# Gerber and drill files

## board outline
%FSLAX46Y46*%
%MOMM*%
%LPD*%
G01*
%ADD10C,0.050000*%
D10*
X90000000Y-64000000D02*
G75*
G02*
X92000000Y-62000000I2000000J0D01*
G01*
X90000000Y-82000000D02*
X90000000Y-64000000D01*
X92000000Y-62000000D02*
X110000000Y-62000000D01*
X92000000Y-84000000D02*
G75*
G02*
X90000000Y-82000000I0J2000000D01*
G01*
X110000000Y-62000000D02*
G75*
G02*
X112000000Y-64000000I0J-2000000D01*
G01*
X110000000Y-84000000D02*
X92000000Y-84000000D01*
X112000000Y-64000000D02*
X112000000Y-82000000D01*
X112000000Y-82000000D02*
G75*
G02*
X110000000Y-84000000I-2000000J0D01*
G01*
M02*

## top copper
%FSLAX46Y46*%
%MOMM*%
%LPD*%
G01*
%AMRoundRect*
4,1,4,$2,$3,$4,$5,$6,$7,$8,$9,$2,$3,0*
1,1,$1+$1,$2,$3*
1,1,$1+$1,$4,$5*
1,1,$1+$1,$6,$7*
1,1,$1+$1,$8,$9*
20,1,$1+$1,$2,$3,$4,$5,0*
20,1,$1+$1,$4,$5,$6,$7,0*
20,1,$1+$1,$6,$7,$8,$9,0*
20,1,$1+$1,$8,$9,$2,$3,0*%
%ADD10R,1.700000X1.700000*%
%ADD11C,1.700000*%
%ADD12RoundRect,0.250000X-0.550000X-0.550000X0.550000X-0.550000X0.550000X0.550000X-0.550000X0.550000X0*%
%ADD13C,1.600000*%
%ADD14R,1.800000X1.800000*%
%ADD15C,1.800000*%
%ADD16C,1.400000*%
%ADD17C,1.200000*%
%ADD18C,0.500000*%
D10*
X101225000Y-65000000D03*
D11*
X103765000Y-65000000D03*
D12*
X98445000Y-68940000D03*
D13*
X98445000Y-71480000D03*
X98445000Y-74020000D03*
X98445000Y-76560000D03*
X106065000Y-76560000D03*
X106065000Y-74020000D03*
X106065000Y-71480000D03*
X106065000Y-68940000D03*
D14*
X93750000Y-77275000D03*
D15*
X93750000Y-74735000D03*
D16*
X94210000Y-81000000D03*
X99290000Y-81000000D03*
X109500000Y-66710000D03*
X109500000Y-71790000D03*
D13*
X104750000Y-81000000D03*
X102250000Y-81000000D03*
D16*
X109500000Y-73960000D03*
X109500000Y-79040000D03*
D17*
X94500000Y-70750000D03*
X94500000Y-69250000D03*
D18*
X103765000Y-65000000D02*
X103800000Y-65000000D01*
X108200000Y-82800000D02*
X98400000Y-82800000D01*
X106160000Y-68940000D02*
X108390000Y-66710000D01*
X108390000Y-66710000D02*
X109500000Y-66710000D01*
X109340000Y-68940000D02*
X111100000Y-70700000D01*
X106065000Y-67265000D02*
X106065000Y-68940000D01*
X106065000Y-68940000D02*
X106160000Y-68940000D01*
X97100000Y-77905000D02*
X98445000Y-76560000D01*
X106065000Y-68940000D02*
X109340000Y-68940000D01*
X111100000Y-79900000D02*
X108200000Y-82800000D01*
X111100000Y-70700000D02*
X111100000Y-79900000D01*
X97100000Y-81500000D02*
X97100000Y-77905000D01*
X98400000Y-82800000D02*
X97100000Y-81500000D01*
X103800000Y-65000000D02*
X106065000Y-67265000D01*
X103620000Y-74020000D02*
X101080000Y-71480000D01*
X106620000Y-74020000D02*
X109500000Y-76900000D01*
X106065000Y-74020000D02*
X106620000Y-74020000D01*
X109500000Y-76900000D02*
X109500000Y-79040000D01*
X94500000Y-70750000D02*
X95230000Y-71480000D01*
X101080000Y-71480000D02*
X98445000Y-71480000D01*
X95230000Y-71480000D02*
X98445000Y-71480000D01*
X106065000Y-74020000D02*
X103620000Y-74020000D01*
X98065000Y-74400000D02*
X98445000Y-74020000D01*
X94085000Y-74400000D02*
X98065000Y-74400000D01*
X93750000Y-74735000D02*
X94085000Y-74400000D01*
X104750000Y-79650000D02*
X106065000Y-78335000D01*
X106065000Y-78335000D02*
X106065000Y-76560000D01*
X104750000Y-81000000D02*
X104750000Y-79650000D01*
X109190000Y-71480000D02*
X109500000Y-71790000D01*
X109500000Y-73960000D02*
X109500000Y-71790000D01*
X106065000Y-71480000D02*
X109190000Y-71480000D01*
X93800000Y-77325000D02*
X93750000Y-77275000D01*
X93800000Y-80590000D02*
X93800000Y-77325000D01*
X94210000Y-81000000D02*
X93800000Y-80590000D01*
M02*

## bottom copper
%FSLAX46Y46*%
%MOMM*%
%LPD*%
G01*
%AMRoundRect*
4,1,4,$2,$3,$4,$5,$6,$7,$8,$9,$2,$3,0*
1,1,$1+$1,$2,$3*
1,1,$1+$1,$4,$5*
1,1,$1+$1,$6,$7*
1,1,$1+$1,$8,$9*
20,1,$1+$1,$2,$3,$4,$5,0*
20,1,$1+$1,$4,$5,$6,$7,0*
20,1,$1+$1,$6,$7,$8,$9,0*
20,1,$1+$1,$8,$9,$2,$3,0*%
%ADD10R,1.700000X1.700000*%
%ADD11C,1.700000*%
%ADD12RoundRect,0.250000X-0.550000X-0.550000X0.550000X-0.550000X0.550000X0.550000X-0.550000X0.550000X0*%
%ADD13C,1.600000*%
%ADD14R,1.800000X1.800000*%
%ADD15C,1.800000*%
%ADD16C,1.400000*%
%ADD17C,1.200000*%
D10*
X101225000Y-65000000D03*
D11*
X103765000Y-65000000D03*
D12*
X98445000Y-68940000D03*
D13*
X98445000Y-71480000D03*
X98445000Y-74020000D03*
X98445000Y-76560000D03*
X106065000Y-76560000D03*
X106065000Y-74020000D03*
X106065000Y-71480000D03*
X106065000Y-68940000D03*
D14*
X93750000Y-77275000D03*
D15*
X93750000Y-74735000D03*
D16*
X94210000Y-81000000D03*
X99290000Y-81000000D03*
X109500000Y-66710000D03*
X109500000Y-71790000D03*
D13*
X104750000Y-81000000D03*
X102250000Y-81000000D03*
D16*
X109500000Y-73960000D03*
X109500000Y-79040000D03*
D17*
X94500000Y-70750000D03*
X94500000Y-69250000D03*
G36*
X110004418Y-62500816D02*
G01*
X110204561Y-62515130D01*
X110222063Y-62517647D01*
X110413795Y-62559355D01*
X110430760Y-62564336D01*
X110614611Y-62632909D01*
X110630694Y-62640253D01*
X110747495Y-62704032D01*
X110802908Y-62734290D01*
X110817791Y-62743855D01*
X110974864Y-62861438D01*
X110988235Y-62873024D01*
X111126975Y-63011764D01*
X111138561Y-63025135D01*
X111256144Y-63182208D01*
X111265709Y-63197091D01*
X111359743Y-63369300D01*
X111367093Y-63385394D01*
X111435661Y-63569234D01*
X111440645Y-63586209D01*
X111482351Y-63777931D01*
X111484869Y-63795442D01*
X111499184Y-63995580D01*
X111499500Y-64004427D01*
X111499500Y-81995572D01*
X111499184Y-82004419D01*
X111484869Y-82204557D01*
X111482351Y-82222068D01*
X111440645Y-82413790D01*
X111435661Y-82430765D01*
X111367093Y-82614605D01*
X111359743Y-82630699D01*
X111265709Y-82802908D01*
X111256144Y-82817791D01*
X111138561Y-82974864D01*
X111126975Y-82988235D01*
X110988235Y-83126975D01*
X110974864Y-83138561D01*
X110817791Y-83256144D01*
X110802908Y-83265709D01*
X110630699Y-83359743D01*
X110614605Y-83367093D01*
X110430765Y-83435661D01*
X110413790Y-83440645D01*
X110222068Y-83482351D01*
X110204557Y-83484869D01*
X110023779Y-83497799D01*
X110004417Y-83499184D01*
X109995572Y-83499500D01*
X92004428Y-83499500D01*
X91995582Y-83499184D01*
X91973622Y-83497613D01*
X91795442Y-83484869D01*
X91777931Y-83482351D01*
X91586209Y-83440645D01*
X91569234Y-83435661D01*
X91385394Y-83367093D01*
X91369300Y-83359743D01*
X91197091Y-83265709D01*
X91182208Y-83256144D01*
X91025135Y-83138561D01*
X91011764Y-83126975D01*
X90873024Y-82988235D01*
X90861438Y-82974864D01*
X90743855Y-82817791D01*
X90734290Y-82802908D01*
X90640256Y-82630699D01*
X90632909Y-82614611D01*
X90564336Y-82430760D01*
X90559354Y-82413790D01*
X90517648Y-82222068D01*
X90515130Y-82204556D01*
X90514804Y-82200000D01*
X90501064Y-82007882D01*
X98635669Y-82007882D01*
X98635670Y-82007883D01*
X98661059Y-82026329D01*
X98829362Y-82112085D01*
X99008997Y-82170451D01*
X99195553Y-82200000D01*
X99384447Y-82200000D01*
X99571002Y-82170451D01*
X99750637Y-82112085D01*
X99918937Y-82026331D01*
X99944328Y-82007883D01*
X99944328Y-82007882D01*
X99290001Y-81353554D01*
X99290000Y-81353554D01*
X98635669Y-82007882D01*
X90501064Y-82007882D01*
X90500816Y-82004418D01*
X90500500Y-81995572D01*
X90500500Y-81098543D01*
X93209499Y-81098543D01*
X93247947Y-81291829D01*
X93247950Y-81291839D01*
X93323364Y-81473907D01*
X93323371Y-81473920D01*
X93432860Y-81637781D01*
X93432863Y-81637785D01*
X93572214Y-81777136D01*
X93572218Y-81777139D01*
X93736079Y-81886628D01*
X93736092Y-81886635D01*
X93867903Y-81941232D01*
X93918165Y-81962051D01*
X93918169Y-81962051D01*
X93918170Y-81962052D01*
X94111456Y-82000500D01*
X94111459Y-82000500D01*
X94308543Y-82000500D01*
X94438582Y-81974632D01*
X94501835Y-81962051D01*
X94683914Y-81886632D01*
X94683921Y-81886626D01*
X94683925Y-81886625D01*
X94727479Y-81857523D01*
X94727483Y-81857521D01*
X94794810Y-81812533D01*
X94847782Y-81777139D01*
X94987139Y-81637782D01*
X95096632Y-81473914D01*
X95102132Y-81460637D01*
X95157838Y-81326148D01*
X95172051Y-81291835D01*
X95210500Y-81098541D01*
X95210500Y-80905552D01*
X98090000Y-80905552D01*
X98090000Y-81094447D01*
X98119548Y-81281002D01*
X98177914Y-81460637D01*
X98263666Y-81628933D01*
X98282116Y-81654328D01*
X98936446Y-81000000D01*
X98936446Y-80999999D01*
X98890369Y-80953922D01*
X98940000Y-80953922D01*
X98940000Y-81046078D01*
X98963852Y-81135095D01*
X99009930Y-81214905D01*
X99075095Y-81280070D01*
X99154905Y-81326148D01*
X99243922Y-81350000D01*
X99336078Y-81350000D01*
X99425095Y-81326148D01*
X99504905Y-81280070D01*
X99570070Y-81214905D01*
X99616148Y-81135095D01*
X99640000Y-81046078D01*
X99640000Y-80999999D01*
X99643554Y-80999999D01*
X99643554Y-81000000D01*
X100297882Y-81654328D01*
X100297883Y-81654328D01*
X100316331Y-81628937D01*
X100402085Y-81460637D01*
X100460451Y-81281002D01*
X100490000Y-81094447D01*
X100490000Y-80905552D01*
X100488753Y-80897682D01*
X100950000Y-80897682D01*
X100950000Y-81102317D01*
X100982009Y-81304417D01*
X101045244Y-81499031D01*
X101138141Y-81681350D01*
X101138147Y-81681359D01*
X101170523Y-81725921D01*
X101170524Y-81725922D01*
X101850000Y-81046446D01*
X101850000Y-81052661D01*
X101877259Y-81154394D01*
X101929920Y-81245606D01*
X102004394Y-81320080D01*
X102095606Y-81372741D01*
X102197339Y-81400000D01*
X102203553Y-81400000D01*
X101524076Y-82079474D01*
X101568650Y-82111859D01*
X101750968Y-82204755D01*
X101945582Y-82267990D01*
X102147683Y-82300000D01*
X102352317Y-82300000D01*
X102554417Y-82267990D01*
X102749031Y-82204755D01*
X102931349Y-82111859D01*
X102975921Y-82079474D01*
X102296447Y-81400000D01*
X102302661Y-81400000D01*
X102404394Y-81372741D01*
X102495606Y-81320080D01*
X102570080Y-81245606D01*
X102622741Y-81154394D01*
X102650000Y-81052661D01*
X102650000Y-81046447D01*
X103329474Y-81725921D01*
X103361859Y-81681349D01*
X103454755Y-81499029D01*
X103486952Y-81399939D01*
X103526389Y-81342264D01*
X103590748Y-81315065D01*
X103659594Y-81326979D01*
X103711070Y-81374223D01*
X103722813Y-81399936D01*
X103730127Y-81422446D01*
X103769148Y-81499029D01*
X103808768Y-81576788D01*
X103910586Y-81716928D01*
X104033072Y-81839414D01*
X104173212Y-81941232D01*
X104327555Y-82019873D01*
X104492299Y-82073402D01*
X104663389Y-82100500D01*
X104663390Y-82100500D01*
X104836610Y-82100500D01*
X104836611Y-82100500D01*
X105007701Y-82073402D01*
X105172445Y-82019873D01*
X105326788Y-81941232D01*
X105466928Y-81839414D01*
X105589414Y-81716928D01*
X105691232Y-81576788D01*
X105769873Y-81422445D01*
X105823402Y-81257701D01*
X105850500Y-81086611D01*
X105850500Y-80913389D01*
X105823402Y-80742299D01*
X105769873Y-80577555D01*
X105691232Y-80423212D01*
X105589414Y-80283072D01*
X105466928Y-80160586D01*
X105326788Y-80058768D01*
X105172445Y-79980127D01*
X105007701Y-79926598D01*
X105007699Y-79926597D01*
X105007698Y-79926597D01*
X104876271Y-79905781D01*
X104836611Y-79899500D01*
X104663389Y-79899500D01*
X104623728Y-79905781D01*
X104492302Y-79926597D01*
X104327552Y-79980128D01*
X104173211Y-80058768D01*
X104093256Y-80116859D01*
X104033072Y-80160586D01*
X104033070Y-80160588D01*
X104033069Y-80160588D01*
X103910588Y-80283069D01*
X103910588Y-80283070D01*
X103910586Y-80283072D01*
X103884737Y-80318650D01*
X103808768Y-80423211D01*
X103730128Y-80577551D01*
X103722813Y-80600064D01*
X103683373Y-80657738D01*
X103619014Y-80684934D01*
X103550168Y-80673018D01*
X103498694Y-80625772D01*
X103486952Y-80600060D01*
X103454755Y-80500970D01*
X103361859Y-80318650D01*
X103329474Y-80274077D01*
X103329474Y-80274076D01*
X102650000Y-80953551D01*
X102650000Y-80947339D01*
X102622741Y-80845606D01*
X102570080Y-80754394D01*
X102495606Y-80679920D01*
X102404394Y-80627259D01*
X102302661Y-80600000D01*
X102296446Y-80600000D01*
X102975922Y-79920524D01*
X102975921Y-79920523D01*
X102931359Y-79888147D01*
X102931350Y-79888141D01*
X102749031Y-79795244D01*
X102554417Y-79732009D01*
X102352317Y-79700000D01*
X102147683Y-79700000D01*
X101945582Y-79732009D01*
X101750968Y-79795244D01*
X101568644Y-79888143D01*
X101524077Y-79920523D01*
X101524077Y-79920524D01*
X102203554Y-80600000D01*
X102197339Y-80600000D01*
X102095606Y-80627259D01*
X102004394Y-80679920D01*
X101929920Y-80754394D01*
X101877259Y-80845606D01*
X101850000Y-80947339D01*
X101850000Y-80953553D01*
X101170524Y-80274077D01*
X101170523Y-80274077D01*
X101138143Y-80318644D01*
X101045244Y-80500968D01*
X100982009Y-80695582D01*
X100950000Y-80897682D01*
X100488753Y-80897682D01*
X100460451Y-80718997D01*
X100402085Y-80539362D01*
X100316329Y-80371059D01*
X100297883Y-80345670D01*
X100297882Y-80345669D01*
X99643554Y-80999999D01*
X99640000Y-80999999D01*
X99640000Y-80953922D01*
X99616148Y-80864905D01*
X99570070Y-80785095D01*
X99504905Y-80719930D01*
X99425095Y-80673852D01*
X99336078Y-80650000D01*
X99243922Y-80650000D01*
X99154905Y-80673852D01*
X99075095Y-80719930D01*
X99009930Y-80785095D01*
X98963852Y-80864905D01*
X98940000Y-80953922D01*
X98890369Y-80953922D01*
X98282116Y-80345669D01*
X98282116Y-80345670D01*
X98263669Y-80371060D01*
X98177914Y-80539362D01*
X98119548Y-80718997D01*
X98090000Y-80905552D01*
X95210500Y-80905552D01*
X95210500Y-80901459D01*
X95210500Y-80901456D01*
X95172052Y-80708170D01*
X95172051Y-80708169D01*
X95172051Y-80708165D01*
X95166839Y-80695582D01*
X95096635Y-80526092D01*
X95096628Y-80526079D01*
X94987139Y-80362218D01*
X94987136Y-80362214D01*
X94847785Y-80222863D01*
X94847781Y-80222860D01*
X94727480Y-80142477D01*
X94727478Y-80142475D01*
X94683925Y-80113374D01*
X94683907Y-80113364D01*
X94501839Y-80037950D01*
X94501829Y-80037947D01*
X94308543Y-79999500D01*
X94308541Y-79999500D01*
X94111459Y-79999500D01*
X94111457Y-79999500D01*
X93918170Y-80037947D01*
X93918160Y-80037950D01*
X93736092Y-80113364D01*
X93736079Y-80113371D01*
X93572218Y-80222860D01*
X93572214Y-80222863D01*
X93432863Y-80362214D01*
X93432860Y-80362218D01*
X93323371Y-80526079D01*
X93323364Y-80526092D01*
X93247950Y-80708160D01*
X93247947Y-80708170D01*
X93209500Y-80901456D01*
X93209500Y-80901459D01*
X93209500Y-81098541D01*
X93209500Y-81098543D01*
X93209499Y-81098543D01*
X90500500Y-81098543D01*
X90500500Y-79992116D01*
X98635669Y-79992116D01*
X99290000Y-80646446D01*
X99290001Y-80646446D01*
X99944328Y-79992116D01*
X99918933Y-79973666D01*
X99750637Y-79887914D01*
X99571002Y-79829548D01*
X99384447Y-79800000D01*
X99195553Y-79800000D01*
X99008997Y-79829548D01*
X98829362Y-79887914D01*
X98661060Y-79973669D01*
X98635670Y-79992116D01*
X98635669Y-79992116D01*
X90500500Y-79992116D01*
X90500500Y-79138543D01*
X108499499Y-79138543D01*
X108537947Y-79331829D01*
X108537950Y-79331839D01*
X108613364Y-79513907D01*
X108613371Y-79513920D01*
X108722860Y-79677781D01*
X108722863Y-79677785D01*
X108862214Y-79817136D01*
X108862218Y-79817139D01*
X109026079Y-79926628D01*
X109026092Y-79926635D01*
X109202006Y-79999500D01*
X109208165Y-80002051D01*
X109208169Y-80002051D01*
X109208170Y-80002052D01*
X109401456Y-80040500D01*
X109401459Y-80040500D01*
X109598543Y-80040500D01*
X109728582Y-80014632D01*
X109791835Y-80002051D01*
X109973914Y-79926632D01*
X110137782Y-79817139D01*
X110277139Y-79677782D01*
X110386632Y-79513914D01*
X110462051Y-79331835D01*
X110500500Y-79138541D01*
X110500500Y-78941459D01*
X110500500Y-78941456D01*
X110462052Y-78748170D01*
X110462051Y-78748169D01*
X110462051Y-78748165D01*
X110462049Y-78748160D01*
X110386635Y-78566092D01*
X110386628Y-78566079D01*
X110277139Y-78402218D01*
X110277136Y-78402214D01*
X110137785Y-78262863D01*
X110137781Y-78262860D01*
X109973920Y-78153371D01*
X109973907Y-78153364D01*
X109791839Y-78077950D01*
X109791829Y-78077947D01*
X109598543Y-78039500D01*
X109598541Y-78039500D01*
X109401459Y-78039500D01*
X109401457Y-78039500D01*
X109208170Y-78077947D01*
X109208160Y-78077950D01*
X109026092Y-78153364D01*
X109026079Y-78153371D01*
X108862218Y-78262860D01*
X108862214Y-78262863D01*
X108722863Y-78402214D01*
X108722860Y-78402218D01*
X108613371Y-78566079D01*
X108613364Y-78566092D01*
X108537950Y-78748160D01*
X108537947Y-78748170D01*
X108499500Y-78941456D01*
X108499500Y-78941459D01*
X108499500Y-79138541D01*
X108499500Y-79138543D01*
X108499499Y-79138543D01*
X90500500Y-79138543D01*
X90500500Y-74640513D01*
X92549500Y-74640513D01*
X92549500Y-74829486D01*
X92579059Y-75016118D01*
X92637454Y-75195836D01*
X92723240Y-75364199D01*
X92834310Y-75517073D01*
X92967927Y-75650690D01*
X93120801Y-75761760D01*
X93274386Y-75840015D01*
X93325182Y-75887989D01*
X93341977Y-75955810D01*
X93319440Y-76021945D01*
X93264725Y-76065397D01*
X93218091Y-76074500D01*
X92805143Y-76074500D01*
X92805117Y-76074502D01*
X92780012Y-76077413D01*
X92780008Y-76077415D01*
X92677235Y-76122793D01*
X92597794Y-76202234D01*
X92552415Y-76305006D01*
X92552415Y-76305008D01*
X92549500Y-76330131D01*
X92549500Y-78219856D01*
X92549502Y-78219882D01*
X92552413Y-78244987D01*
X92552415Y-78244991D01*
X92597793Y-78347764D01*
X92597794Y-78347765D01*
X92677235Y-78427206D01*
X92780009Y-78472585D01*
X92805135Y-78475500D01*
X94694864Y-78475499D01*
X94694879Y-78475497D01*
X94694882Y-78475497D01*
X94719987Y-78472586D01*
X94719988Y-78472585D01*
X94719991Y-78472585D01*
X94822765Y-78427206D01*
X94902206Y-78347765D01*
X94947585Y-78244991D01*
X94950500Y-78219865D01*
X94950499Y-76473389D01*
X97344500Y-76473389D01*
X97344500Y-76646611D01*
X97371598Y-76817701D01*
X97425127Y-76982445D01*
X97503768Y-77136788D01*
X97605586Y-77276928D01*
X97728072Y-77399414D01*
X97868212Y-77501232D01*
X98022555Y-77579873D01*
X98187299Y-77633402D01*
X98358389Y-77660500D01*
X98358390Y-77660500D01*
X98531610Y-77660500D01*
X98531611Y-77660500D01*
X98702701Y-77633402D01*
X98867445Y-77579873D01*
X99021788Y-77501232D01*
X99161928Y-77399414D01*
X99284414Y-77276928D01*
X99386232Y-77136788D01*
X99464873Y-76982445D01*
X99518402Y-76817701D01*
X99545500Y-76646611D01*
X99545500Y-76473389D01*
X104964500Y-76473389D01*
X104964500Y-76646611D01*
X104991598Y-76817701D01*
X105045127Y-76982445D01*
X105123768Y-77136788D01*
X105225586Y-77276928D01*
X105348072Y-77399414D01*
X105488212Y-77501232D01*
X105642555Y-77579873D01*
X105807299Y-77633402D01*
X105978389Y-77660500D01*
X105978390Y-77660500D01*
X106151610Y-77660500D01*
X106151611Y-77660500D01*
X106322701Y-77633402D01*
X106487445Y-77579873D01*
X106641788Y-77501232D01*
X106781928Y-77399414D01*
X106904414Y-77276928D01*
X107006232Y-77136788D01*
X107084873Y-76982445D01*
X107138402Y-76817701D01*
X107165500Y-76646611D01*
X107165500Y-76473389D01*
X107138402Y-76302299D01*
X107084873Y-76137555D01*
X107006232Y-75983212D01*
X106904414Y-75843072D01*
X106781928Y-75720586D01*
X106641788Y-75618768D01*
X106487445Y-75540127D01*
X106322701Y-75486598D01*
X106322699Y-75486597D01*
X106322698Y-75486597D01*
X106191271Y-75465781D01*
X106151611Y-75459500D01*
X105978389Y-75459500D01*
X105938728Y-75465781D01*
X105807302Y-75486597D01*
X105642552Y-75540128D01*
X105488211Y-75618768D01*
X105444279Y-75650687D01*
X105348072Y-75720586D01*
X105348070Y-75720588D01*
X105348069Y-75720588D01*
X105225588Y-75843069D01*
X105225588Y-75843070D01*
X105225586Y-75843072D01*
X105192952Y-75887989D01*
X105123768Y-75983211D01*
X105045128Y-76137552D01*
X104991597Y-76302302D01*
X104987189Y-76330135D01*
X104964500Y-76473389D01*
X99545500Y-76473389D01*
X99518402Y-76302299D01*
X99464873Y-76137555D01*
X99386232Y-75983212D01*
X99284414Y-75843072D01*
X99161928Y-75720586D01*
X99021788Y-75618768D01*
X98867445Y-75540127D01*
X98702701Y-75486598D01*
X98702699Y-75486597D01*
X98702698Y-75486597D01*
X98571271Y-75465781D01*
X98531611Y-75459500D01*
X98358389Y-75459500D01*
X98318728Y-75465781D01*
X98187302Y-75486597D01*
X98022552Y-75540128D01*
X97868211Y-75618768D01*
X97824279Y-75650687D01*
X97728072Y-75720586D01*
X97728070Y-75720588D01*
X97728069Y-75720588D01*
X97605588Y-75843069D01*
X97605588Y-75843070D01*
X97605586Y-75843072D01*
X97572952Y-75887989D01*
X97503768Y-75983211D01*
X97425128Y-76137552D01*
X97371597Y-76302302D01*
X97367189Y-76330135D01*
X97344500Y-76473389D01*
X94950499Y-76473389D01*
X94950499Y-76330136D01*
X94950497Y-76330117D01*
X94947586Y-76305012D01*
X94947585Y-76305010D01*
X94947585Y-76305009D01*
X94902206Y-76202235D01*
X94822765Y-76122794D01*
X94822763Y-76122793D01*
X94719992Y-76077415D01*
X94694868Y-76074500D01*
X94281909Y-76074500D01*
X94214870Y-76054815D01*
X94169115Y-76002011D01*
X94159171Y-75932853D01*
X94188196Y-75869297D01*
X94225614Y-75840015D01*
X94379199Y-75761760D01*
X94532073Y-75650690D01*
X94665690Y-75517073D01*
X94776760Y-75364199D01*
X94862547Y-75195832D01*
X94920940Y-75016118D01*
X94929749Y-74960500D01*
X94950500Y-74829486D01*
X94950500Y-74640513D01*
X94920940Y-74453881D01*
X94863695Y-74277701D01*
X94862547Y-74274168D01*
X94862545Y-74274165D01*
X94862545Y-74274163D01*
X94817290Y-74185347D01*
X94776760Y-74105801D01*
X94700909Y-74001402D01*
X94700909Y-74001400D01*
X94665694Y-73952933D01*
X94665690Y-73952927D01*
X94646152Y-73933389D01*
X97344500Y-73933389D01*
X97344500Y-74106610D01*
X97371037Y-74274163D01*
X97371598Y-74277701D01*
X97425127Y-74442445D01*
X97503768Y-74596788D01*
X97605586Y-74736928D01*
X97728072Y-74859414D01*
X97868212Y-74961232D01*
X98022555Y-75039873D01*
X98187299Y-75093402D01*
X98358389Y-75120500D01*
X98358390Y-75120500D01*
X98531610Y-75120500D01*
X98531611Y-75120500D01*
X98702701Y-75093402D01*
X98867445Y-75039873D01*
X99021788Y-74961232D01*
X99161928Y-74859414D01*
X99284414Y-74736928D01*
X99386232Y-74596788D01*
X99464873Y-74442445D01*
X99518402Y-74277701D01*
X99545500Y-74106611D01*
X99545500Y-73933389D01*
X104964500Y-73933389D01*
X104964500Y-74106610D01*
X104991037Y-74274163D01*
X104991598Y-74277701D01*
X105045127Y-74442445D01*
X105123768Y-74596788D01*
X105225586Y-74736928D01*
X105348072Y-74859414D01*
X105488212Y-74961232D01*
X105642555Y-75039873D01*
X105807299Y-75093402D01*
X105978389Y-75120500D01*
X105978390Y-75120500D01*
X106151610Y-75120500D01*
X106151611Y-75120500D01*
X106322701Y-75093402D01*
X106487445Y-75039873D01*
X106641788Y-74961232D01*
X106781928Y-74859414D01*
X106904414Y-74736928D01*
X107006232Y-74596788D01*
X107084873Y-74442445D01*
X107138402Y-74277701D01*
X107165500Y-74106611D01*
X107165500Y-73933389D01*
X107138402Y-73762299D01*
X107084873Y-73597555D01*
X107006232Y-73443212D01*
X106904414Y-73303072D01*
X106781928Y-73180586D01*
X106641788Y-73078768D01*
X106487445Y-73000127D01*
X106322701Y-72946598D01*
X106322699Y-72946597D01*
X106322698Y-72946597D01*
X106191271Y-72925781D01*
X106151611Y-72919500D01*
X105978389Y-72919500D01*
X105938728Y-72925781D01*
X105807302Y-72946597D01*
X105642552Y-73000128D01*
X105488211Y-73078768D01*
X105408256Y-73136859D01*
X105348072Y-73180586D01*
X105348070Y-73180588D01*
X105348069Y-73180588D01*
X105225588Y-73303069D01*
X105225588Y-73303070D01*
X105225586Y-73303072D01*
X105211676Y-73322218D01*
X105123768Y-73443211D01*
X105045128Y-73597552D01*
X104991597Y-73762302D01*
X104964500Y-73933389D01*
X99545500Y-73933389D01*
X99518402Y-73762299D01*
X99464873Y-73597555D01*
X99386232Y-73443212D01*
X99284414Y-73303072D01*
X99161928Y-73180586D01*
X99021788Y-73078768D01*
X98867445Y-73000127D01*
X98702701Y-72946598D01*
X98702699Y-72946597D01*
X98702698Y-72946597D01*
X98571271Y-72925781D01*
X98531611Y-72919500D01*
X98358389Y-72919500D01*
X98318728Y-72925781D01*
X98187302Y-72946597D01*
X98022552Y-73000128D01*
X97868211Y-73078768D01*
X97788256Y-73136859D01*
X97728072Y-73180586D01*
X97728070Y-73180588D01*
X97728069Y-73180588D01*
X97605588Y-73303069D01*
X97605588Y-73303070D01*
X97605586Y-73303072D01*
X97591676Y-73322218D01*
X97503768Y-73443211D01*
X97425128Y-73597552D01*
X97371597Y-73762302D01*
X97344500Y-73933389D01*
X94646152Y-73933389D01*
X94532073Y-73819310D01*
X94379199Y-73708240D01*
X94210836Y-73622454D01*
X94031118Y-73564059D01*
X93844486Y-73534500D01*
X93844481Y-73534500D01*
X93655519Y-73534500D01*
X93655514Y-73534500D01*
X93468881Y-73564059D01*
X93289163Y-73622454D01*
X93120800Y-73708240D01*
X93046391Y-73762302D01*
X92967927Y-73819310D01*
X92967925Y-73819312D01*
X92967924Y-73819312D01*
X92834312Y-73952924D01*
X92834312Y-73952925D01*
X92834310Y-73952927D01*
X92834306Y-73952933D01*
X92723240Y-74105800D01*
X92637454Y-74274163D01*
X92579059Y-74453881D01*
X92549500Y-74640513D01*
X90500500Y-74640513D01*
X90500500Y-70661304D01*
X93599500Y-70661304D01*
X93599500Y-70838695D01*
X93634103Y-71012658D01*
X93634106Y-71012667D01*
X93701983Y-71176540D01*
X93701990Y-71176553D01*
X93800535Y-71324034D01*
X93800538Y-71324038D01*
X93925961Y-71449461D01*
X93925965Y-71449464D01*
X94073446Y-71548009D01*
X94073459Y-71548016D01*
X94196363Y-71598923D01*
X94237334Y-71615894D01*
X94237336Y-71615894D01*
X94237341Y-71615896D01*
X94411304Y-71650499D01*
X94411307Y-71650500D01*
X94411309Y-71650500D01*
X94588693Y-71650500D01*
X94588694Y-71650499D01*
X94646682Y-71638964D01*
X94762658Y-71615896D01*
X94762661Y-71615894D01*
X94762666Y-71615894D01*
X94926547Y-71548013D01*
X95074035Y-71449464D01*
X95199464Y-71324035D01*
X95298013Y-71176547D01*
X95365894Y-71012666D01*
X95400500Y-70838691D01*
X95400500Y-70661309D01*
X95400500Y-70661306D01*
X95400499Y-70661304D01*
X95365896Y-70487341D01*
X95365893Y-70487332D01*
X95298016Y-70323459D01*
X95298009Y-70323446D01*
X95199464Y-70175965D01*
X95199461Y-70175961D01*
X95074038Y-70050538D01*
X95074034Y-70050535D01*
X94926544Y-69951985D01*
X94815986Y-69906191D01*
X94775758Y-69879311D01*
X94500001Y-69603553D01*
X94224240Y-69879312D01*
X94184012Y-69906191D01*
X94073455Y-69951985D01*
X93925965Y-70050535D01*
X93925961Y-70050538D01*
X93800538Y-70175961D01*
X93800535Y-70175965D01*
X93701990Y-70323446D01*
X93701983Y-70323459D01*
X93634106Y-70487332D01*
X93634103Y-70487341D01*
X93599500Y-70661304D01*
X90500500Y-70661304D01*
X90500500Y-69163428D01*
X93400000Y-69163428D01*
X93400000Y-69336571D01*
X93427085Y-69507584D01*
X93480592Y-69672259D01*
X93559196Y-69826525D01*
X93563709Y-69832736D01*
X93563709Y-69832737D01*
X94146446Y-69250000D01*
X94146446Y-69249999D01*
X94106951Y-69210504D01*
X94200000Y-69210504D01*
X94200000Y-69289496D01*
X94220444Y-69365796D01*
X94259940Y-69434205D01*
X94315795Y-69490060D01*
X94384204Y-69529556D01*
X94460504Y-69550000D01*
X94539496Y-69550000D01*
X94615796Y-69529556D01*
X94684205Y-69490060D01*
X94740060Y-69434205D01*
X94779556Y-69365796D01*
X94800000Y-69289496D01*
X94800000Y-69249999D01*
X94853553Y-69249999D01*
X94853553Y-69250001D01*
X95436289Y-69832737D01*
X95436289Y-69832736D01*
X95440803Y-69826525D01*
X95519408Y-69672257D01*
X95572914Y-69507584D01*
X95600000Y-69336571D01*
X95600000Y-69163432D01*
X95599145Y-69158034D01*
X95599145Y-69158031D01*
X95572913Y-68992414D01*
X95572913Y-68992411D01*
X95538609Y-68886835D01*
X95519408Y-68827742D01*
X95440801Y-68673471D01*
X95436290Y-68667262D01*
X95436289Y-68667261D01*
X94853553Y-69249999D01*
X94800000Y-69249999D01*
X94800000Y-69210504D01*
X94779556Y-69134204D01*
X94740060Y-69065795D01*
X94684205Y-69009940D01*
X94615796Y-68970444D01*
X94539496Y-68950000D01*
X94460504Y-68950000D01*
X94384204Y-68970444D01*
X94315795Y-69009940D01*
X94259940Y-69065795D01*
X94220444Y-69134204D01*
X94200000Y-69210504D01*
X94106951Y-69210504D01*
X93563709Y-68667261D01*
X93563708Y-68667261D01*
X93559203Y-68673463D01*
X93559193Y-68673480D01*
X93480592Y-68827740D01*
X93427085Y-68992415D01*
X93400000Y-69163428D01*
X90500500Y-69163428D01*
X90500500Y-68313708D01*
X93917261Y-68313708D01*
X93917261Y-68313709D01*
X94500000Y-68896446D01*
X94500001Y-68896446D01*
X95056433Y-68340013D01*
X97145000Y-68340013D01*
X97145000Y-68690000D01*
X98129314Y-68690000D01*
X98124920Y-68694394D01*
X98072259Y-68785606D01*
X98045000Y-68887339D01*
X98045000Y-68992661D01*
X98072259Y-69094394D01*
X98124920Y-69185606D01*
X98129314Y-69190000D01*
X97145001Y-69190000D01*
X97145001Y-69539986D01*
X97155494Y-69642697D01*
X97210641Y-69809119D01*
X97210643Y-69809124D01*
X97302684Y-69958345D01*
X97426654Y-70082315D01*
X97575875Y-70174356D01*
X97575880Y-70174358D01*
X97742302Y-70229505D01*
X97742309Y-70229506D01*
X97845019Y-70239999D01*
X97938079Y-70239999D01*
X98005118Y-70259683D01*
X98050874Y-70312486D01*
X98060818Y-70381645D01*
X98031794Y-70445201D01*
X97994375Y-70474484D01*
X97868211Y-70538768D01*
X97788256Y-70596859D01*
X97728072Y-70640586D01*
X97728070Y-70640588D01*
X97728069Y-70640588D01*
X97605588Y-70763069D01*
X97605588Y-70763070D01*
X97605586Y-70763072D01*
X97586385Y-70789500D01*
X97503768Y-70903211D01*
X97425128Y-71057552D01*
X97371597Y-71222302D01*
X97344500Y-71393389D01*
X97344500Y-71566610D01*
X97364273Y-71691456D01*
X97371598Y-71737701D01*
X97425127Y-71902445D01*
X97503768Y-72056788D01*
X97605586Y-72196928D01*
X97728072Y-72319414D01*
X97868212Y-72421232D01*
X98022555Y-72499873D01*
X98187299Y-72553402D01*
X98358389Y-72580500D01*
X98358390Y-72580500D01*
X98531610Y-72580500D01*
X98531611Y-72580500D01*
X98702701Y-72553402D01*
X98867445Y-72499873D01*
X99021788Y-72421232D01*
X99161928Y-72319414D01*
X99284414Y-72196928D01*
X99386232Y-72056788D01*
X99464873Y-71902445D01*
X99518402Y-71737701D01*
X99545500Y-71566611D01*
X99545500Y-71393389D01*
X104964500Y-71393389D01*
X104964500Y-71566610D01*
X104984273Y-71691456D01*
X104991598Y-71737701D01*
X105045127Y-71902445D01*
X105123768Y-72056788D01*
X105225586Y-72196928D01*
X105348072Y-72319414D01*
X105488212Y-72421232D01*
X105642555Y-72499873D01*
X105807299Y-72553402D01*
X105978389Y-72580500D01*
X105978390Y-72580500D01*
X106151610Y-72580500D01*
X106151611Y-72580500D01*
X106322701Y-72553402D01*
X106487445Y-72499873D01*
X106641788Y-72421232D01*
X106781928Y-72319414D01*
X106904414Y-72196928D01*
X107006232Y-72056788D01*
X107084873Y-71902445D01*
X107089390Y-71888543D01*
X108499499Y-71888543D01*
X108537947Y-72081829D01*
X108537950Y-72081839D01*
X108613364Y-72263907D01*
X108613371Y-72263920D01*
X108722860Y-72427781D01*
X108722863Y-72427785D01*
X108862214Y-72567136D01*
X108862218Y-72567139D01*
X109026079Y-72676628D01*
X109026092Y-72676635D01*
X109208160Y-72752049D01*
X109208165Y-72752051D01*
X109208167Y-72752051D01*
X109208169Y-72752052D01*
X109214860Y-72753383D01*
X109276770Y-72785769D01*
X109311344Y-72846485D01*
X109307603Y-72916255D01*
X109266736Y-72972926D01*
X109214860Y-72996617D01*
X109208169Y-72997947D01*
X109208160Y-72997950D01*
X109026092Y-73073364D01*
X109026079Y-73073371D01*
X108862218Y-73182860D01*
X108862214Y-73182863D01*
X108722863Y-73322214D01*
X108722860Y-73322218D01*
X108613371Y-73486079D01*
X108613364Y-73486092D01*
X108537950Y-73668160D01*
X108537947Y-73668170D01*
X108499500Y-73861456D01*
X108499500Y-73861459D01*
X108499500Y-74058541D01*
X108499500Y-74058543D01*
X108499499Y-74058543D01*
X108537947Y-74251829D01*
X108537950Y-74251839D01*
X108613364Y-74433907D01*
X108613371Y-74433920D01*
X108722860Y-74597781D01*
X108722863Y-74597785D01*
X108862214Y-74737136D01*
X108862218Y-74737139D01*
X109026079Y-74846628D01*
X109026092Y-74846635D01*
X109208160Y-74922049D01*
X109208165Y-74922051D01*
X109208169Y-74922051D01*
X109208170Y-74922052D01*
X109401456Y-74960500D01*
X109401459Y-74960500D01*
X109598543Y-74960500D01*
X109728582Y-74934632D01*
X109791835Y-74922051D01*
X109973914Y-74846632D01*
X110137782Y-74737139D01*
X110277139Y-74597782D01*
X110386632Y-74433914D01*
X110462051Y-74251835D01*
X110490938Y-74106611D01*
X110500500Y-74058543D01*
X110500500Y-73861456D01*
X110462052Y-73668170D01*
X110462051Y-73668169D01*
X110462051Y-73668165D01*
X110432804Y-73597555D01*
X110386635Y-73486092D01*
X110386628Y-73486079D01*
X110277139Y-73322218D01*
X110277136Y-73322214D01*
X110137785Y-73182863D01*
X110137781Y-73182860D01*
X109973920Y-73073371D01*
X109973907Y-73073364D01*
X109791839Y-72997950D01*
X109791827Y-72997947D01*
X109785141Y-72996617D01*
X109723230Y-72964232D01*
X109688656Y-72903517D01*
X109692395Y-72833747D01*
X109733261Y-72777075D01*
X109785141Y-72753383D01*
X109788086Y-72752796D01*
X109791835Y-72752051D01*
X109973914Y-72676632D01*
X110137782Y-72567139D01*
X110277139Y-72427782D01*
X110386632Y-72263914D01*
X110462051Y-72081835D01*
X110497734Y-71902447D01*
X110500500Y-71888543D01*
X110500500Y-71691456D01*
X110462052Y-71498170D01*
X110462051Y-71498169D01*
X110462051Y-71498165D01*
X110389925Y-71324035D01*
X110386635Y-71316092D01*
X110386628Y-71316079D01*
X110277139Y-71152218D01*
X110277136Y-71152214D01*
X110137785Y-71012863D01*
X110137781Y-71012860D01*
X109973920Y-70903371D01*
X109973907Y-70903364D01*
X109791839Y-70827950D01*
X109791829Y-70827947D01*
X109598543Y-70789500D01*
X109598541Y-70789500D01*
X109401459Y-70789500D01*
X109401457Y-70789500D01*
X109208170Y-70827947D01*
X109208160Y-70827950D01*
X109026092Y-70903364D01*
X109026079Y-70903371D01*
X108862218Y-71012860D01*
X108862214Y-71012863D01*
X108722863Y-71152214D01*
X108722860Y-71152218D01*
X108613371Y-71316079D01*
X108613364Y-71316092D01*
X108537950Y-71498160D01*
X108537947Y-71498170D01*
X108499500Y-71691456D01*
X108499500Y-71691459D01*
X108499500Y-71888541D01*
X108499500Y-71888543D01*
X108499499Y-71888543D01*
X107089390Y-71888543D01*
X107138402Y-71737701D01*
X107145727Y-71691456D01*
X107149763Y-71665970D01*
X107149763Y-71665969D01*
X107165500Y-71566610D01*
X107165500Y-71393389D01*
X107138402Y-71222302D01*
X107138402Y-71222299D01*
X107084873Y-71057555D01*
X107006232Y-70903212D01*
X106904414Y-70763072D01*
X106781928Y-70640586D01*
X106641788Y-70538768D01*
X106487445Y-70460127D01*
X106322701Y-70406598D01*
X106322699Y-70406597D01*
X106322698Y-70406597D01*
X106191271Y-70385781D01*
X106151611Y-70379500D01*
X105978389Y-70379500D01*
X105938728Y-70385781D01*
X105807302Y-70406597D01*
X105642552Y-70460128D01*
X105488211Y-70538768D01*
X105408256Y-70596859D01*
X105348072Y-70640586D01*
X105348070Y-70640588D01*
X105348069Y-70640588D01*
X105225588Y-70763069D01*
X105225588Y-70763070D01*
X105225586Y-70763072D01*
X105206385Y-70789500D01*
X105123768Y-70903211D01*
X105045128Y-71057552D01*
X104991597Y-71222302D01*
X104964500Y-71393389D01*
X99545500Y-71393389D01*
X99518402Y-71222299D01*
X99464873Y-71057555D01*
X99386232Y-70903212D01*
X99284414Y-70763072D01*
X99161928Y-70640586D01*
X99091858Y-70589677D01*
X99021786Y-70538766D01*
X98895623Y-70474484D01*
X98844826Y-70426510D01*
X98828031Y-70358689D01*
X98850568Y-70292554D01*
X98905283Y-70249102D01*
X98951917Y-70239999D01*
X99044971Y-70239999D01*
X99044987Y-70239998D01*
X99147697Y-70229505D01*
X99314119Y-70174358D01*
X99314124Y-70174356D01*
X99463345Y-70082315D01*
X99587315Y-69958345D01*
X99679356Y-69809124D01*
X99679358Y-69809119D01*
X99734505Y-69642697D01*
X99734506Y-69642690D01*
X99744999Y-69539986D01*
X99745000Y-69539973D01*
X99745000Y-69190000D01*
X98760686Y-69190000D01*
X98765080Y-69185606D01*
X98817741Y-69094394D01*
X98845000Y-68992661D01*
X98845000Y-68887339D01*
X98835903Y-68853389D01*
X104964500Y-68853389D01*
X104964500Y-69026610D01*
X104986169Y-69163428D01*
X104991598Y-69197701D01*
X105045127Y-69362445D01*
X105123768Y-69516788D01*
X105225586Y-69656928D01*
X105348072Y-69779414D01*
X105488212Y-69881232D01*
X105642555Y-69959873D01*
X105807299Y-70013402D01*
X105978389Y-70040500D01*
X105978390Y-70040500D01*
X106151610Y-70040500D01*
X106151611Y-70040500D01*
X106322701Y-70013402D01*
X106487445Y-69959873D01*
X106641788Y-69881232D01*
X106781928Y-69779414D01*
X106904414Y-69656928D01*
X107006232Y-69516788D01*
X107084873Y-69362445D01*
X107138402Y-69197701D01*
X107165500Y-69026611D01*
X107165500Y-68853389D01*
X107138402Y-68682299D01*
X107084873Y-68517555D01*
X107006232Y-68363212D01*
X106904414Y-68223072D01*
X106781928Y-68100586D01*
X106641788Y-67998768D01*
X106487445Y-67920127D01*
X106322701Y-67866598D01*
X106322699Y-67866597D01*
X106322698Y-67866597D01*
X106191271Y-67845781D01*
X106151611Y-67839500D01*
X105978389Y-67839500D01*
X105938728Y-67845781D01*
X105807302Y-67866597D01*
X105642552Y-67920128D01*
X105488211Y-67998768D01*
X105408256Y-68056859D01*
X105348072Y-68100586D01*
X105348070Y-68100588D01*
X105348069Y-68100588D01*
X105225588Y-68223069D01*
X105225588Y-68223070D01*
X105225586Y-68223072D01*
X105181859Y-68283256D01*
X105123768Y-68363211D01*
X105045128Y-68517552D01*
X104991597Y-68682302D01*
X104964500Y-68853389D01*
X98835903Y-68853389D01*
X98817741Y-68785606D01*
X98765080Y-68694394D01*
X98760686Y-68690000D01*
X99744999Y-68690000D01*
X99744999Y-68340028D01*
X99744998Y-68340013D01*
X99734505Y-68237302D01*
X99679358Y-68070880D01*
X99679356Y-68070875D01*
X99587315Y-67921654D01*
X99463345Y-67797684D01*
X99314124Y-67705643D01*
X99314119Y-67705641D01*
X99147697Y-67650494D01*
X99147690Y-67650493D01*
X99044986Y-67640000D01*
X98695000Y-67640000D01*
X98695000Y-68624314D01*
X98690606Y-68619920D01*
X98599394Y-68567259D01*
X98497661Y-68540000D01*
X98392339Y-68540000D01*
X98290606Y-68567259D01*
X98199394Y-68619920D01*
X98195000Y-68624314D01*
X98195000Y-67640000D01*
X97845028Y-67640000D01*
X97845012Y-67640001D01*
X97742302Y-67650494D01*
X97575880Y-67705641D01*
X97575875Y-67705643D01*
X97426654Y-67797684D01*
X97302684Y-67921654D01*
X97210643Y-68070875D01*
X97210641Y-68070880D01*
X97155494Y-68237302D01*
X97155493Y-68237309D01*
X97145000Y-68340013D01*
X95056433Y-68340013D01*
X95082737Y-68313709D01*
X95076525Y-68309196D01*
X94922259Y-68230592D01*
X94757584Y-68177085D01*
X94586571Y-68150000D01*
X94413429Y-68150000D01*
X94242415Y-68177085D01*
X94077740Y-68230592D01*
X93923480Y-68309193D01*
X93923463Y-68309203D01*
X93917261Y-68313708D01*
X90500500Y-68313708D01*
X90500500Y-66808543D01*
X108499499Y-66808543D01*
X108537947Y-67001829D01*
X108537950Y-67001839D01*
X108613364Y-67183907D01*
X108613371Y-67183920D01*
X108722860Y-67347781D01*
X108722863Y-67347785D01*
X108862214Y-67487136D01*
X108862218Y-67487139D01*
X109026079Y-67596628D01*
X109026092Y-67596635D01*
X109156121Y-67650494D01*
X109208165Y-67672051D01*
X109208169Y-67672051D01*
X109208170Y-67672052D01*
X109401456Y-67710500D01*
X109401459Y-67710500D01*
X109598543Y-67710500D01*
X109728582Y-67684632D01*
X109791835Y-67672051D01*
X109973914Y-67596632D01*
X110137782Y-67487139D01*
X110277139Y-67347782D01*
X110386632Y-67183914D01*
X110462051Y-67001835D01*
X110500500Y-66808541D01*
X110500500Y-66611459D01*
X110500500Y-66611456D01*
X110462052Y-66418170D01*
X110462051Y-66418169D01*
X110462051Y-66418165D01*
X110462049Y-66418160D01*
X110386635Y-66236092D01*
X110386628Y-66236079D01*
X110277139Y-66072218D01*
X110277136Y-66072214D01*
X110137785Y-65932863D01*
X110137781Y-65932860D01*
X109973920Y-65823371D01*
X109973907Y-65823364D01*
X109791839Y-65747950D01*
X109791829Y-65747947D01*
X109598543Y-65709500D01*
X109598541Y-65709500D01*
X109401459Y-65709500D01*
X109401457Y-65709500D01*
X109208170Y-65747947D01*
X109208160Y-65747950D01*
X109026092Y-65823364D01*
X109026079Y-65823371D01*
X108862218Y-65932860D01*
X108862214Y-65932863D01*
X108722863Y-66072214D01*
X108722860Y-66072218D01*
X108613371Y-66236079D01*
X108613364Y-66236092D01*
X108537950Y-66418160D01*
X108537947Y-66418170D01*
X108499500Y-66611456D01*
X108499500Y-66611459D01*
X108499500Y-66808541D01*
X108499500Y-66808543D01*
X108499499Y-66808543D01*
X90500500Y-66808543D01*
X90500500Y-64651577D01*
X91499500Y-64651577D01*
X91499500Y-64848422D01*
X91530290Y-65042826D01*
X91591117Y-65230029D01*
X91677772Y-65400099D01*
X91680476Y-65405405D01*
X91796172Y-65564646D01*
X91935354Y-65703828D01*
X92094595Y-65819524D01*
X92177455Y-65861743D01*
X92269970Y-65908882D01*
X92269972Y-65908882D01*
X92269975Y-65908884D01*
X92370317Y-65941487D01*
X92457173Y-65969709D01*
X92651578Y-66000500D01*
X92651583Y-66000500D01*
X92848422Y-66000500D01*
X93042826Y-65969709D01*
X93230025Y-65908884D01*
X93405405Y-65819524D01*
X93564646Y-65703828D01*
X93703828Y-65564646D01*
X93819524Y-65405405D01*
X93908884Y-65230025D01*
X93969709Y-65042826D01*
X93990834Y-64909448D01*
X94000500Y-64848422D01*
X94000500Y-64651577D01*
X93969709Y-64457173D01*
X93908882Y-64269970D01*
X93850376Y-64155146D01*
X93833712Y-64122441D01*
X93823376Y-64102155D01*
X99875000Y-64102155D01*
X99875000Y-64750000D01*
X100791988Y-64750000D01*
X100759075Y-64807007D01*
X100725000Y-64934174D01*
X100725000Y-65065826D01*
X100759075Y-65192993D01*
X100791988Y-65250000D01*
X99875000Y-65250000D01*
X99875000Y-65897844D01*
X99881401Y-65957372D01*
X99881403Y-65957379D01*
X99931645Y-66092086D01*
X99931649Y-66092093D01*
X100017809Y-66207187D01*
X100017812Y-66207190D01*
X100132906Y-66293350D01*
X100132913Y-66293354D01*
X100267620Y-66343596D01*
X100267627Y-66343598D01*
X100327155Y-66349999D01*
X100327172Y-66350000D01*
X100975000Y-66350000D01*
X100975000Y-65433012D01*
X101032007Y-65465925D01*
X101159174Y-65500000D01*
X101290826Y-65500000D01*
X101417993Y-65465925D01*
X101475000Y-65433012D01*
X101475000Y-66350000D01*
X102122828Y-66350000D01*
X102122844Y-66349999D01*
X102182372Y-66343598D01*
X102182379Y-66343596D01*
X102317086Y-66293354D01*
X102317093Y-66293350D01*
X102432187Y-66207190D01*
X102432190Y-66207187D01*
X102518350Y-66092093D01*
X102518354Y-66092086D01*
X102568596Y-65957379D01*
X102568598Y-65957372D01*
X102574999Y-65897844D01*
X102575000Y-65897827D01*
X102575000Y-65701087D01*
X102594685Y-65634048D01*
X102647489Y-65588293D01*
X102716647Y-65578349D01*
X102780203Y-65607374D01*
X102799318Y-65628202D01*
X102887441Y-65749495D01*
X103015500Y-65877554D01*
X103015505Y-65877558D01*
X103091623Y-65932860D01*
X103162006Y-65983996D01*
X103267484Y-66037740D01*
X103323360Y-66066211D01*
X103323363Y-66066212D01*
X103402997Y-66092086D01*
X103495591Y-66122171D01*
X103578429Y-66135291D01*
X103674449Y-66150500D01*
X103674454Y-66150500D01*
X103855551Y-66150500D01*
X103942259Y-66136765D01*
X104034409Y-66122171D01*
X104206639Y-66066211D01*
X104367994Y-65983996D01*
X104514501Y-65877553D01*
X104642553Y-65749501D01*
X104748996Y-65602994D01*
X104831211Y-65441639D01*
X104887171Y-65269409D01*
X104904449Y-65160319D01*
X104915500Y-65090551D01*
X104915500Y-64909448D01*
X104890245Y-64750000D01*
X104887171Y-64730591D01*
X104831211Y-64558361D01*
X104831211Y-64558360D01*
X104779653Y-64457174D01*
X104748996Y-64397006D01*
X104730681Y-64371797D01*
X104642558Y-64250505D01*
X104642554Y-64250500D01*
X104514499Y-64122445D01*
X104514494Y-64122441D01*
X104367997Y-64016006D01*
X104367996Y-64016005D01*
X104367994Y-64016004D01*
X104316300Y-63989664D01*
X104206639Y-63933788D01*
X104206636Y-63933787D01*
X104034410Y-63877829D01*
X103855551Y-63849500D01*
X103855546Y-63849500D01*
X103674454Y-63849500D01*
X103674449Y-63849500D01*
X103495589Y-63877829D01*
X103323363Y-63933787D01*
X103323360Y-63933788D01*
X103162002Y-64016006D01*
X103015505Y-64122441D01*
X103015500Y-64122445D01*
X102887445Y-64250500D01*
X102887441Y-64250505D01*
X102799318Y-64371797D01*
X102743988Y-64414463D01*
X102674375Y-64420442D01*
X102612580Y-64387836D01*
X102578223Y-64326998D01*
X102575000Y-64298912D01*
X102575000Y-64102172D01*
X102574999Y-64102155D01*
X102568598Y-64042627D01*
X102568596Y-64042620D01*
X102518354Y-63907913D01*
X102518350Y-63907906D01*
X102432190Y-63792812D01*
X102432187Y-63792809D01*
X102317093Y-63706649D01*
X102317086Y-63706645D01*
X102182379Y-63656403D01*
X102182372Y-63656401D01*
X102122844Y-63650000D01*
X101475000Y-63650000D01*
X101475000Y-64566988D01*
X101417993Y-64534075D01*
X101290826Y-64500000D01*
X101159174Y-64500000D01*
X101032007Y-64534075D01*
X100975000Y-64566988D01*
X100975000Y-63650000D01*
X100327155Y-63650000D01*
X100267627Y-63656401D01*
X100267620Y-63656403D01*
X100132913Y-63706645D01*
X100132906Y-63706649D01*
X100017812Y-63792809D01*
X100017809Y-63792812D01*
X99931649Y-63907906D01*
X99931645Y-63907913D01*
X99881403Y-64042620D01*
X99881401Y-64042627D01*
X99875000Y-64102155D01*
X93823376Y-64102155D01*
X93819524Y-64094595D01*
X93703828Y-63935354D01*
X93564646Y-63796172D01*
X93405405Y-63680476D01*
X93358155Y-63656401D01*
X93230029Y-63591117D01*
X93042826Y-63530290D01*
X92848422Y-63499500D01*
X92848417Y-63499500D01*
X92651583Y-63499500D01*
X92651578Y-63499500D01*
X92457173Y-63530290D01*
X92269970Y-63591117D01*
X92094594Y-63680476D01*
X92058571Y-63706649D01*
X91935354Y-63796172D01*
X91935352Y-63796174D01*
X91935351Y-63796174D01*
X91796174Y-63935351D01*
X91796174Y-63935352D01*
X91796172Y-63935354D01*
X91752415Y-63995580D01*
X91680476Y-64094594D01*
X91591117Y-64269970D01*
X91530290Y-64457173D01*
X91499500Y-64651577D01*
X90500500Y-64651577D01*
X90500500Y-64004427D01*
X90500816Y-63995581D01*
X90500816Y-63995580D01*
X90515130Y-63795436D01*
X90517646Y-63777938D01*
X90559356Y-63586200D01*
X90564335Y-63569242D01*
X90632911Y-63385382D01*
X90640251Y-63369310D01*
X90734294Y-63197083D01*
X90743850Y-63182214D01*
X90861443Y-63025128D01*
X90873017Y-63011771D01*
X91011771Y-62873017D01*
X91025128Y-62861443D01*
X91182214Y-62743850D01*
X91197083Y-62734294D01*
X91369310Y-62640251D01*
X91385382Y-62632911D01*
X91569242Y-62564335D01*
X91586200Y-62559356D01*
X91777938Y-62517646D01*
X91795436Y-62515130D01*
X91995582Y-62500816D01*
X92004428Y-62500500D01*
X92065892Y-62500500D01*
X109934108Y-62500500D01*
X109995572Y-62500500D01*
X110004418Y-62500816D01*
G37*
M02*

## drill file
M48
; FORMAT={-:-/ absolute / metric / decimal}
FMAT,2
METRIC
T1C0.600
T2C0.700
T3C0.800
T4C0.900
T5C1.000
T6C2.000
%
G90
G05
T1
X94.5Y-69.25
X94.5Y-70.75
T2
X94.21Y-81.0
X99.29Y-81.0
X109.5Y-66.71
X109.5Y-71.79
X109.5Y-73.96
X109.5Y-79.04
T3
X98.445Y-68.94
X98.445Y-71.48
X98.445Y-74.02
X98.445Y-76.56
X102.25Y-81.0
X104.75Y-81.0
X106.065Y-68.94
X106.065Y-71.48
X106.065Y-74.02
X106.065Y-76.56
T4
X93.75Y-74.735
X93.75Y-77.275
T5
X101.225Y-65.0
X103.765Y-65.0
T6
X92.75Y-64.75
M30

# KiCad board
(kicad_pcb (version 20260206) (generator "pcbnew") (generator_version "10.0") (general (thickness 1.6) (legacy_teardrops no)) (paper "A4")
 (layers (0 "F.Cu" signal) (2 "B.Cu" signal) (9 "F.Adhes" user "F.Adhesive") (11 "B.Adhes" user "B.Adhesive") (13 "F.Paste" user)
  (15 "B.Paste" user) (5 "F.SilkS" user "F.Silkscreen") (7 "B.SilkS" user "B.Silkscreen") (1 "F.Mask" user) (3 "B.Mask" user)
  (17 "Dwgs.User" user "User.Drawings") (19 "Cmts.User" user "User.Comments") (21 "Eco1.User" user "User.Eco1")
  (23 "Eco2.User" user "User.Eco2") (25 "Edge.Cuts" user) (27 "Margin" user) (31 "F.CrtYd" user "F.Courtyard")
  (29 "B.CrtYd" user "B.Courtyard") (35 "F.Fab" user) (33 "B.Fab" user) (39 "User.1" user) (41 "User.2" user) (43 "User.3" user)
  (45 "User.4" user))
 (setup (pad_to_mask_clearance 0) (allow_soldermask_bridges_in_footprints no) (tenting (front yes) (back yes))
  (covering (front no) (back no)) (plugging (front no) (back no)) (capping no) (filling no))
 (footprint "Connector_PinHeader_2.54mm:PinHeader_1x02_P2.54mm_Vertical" (layer "F.Cu") (at 101.225 65 90)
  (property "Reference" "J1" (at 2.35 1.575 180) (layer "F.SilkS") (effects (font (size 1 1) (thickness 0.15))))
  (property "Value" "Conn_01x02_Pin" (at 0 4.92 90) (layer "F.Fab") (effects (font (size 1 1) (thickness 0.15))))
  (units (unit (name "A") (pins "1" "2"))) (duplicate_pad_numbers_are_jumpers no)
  (pad "1" thru_hole rect (at 0 0 90) (size 1.7 1.7) (drill 1) (layers "*.Cu" "*.Mask") (remove_unused_layers no) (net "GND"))
  (pad "2" thru_hole circle (at 0 2.54 90) (size 1.7 1.7) (drill 1) (layers "*.Cu" "*.Mask") (remove_unused_layers no) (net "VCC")))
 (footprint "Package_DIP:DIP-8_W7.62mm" (layer "F.Cu") (at 98.445 68.94)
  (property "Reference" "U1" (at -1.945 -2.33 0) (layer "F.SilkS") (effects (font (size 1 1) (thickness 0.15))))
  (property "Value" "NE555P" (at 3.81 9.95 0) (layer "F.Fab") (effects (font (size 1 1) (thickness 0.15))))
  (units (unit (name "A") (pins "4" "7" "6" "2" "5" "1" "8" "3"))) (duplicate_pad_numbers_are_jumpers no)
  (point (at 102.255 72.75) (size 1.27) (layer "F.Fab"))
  (pad "1" thru_hole roundrect (at 0 0) (size 1.6 1.6) (drill 0.8) (layers "*.Cu" "*.Mask") (remove_unused_layers no)
   (roundrect_rratio 0.15625) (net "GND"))
  (pad "2" thru_hole circle (at 0 2.54) (size 1.6 1.6) (drill 0.8) (layers "*.Cu" "*.Mask") (remove_unused_layers no) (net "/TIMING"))
  (pad "3" thru_hole circle (at 0 5.08) (size 1.6 1.6) (drill 0.8) (layers "*.Cu" "*.Mask") (remove_unused_layers no) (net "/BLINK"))
  (pad "4" thru_hole circle (at 0 7.62) (size 1.6 1.6) (drill 0.8) (layers "*.Cu" "*.Mask") (remove_unused_layers no) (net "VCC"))
  (pad "5" thru_hole circle (at 7.62 7.62) (size 1.6 1.6) (drill 0.8) (layers "*.Cu" "*.Mask") (remove_unused_layers no)
   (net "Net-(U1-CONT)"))
  (pad "6" thru_hole circle (at 7.62 5.08) (size 1.6 1.6) (drill 0.8) (layers "*.Cu" "*.Mask") (remove_unused_layers no) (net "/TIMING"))
  (pad "7" thru_hole circle (at 7.62 2.54) (size 1.6 1.6) (drill 0.8) (layers "*.Cu" "*.Mask") (remove_unused_layers no) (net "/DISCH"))
  (pad "8" thru_hole circle (at 7.62 0) (size 1.6 1.6) (drill 0.8) (layers "*.Cu" "*.Mask") (remove_unused_layers no) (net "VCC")))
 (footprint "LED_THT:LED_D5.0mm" (layer "F.Cu") (at 93.75 77.275 90)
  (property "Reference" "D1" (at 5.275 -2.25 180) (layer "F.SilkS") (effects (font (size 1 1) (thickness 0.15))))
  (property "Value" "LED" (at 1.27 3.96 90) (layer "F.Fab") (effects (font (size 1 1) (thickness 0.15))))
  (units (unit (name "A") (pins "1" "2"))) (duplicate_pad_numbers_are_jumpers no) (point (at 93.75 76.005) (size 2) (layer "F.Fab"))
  (pad "1" thru_hole rect (at 0 0 90) (size 1.8 1.8) (drill 0.9) (layers "*.Cu" "*.Mask") (remove_unused_layers no) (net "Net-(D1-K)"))
  (pad "2" thru_hole circle (at 2.54 0 90) (size 1.8 1.8) (drill 0.9) (layers "*.Cu" "*.Mask") (remove_unused_layers no) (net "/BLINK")))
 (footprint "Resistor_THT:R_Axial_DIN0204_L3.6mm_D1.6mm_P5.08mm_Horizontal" (layer "F.Cu") (at 94.21 81)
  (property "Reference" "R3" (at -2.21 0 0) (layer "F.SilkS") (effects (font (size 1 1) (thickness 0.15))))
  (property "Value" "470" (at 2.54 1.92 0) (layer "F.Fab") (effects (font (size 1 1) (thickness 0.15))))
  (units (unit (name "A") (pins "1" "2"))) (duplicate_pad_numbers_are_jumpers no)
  (pad "1" thru_hole circle (at 0 0) (size 1.4 1.4) (drill 0.7) (layers "*.Cu" "*.Mask") (remove_unused_layers no) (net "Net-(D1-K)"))
  (pad "2" thru_hole circle (at 5.08 0) (size 1.4 1.4) (drill 0.7) (layers "*.Cu" "*.Mask") (remove_unused_layers no) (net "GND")))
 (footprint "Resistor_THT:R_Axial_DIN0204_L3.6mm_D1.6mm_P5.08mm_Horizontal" (layer "F.Cu") (at 109.5 66.71 -90)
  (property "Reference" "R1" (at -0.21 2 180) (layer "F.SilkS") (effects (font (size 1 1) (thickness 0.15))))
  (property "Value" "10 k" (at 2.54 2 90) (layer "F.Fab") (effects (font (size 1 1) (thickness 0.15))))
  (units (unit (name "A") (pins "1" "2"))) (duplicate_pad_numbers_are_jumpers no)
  (pad "1" thru_hole circle (at 0 0 270) (size 1.4 1.4) (drill 0.7) (layers "*.Cu" "*.Mask") (remove_unused_layers no) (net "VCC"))
  (pad "2" thru_hole circle (at 5.08 0 270) (size 1.4 1.4) (drill 0.7) (layers "*.Cu" "*.Mask") (remove_unused_layers no) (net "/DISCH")))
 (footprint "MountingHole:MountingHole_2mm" (layer "F.Cu") (at 92.75 64.75)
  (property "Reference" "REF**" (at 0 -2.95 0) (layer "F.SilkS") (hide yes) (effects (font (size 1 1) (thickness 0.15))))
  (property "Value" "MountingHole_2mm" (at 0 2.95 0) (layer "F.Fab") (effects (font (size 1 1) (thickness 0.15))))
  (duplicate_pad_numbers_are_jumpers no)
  (pad "" np_thru_hole circle (at 0 0) (size 2 2) (drill 2) (layers "*.Cu" "*.Mask")))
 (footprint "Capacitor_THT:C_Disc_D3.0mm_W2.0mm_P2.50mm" (layer "F.Cu") (at 104.75 81 180)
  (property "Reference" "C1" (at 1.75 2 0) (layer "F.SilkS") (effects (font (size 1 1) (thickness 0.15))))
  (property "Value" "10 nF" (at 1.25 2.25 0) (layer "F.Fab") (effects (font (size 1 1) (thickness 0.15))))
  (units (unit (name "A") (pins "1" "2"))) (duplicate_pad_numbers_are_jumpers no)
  (pad "1" thru_hole circle (at 0 0 180) (size 1.6 1.6) (drill 0.8) (layers "*.Cu" "*.Mask") (remove_unused_layers no) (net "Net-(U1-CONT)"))
  (pad "2" thru_hole circle (at 2.5 0 180) (size 1.6 1.6) (drill 0.8) (layers "*.Cu" "*.Mask") (remove_unused_layers no) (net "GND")))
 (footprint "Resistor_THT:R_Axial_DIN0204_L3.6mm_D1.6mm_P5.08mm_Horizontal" (layer "F.Cu") (at 109.5 73.96 -90)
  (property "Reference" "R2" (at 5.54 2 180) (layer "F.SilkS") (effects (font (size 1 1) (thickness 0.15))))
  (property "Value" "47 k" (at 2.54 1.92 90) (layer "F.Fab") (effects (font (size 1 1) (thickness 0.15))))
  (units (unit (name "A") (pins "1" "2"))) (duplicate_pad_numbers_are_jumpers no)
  (pad "1" thru_hole circle (at 0 0 270) (size 1.4 1.4) (drill 0.7) (layers "*.Cu" "*.Mask") (remove_unused_layers no) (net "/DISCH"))
  (pad "2" thru_hole circle (at 5.08 0 270) (size 1.4 1.4) (drill 0.7) (layers "*.Cu" "*.Mask") (remove_unused_layers no) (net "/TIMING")))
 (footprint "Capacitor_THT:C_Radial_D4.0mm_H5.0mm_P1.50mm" (layer "F.Cu") (at 94.5 70.75 90)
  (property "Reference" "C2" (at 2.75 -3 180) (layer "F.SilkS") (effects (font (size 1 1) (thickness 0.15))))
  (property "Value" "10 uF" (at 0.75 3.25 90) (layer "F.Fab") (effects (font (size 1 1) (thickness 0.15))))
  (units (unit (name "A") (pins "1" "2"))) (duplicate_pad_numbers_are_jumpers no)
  (pad "1" thru_hole circle (at 0 0 90) (size 1.2 1.2) (drill 0.6) (layers "*.Cu" "*.Mask") (remove_unused_layers no) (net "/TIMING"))
  (pad "2" thru_hole circle (at 1.5 0 90) (size 1.2 1.2) (drill 0.6) (layers "*.Cu" "*.Mask") (remove_unused_layers no) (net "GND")))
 (gr_arc (start 90 64) (mid 90.585786 62.585786) (end 92 62) (stroke (width 0.05) (type default)) (layer "Edge.Cuts"))
 (gr_line (start 90 82) (end 90 64) (stroke (width 0.05) (type default)) (layer "Edge.Cuts"))
 (gr_line (start 92 62) (end 110 62) (stroke (width 0.05) (type default)) (layer "Edge.Cuts"))
 (gr_arc (start 92 84) (mid 90.585786 83.414214) (end 90 82) (stroke (width 0.05) (type default)) (layer "Edge.Cuts"))
 (gr_arc (start 110 62) (mid 111.414214 62.585786) (end 112 64) (stroke (width 0.05) (type default)) (layer "Edge.Cuts"))
 (gr_line (start 110 84) (end 92 84) (stroke (width 0.05) (type default)) (layer "Edge.Cuts"))
 (gr_line (start 112 64) (end 112 82) (stroke (width 0.05) (type default)) (layer "Edge.Cuts"))
 (gr_arc (start 112 82) (mid 111.414214 83.414214) (end 110 84) (stroke (width 0.05) (type default)) (layer "Edge.Cuts"))
 (segment (start 103.765 65) (end 103.8 65) (width 0.5) (layer "F.Cu") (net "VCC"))
 (segment (start 108.2 82.8) (end 98.4 82.8) (width 0.5) (layer "F.Cu") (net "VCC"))
 (segment (start 106.16 68.94) (end 108.39 66.71) (width 0.5) (layer "F.Cu") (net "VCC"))
 (segment (start 108.39 66.71) (end 109.5 66.71) (width 0.5) (layer "F.Cu") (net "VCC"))
 (segment (start 109.34 68.94) (end 111.1 70.7) (width 0.5) (layer "F.Cu") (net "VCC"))
 (segment (start 106.065 67.265) (end 106.065 68.94) (width 0.5) (layer "F.Cu") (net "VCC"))
 (segment (start 106.065 68.94) (end 106.16 68.94) (width 0.5) (layer "F.Cu") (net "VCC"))
 (segment (start 97.1 77.905) (end 98.445 76.56) (width 0.5) (layer "F.Cu") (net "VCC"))
 (segment (start 106.065 68.94) (end 109.34 68.94) (width 0.5) (layer "F.Cu") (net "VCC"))
 (segment (start 111.1 79.9) (end 108.2 82.8) (width 0.5) (layer "F.Cu") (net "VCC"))
 (segment (start 111.1 70.7) (end 111.1 79.9) (width 0.5) (layer "F.Cu") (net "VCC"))
 (segment (start 97.1 81.5) (end 97.1 77.905) (width 0.5) (layer "F.Cu") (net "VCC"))
 (segment (start 98.4 82.8) (end 97.1 81.5) (width 0.5) (layer "F.Cu") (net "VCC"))
 (segment (start 103.8 65) (end 106.065 67.265) (width 0.5) (layer "F.Cu") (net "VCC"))
 (segment (start 103.62 74.02) (end 101.08 71.48) (width 0.5) (layer "F.Cu") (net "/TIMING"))
 (segment (start 106.62 74.02) (end 109.5 76.9) (width 0.5) (layer "F.Cu") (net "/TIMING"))
 (segment (start 106.065 74.02) (end 106.62 74.02) (width 0.5) (layer "F.Cu") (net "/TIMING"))
 (segment (start 109.5 76.9) (end 109.5 79.04) (width 0.5) (layer "F.Cu") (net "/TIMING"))
 (segment (start 94.5 70.75) (end 95.23 71.48) (width 0.5) (layer "F.Cu") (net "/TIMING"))
 (segment (start 101.08 71.48) (end 98.445 71.48) (width 0.5) (layer "F.Cu") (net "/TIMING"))
 (segment (start 95.23 71.48) (end 98.445 71.48) (width 0.5) (layer "F.Cu") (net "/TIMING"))
 (segment (start 106.065 74.02) (end 103.62 74.02) (width 0.5) (layer "F.Cu") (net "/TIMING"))
 (segment (start 98.065 74.4) (end 98.445 74.02) (width 0.5) (layer "F.Cu") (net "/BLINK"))
 (segment (start 94.085 74.4) (end 98.065 74.4) (width 0.5) (layer "F.Cu") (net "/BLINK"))
 (segment (start 93.75 74.735) (end 94.085 74.4) (width 0.5) (layer "F.Cu") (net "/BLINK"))
 (segment (start 104.75 79.65) (end 106.065 78.335) (width 0.5) (layer "F.Cu") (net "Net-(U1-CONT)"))
 (segment (start 106.065 78.335) (end 106.065 76.56) (width 0.5) (layer "F.Cu") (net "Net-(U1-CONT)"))
 (segment (start 104.75 81) (end 104.75 79.65) (width 0.5) (layer "F.Cu") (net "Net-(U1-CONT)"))
 (segment (start 109.19 71.48) (end 109.5 71.79) (width 0.5) (layer "F.Cu") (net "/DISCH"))
 (segment (start 109.5 73.96) (end 109.5 71.79) (width 0.5) (layer "F.Cu") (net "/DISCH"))
 (segment (start 106.065 71.48) (end 109.19 71.48) (width 0.5) (layer "F.Cu") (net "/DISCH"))
 (segment (start 93.8 77.325) (end 93.75 77.275) (width 0.5) (layer "F.Cu") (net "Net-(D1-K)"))
 (segment (start 93.8 80.59) (end 93.8 77.325) (width 0.5) (layer "F.Cu") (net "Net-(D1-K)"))
 (segment (start 94.21 81) (end 93.8 80.59) (width 0.5) (layer "F.Cu") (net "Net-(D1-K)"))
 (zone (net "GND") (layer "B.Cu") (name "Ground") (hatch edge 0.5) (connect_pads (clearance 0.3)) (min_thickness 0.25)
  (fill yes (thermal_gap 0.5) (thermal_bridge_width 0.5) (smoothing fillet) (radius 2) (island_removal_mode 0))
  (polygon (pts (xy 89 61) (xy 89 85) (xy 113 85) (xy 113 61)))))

